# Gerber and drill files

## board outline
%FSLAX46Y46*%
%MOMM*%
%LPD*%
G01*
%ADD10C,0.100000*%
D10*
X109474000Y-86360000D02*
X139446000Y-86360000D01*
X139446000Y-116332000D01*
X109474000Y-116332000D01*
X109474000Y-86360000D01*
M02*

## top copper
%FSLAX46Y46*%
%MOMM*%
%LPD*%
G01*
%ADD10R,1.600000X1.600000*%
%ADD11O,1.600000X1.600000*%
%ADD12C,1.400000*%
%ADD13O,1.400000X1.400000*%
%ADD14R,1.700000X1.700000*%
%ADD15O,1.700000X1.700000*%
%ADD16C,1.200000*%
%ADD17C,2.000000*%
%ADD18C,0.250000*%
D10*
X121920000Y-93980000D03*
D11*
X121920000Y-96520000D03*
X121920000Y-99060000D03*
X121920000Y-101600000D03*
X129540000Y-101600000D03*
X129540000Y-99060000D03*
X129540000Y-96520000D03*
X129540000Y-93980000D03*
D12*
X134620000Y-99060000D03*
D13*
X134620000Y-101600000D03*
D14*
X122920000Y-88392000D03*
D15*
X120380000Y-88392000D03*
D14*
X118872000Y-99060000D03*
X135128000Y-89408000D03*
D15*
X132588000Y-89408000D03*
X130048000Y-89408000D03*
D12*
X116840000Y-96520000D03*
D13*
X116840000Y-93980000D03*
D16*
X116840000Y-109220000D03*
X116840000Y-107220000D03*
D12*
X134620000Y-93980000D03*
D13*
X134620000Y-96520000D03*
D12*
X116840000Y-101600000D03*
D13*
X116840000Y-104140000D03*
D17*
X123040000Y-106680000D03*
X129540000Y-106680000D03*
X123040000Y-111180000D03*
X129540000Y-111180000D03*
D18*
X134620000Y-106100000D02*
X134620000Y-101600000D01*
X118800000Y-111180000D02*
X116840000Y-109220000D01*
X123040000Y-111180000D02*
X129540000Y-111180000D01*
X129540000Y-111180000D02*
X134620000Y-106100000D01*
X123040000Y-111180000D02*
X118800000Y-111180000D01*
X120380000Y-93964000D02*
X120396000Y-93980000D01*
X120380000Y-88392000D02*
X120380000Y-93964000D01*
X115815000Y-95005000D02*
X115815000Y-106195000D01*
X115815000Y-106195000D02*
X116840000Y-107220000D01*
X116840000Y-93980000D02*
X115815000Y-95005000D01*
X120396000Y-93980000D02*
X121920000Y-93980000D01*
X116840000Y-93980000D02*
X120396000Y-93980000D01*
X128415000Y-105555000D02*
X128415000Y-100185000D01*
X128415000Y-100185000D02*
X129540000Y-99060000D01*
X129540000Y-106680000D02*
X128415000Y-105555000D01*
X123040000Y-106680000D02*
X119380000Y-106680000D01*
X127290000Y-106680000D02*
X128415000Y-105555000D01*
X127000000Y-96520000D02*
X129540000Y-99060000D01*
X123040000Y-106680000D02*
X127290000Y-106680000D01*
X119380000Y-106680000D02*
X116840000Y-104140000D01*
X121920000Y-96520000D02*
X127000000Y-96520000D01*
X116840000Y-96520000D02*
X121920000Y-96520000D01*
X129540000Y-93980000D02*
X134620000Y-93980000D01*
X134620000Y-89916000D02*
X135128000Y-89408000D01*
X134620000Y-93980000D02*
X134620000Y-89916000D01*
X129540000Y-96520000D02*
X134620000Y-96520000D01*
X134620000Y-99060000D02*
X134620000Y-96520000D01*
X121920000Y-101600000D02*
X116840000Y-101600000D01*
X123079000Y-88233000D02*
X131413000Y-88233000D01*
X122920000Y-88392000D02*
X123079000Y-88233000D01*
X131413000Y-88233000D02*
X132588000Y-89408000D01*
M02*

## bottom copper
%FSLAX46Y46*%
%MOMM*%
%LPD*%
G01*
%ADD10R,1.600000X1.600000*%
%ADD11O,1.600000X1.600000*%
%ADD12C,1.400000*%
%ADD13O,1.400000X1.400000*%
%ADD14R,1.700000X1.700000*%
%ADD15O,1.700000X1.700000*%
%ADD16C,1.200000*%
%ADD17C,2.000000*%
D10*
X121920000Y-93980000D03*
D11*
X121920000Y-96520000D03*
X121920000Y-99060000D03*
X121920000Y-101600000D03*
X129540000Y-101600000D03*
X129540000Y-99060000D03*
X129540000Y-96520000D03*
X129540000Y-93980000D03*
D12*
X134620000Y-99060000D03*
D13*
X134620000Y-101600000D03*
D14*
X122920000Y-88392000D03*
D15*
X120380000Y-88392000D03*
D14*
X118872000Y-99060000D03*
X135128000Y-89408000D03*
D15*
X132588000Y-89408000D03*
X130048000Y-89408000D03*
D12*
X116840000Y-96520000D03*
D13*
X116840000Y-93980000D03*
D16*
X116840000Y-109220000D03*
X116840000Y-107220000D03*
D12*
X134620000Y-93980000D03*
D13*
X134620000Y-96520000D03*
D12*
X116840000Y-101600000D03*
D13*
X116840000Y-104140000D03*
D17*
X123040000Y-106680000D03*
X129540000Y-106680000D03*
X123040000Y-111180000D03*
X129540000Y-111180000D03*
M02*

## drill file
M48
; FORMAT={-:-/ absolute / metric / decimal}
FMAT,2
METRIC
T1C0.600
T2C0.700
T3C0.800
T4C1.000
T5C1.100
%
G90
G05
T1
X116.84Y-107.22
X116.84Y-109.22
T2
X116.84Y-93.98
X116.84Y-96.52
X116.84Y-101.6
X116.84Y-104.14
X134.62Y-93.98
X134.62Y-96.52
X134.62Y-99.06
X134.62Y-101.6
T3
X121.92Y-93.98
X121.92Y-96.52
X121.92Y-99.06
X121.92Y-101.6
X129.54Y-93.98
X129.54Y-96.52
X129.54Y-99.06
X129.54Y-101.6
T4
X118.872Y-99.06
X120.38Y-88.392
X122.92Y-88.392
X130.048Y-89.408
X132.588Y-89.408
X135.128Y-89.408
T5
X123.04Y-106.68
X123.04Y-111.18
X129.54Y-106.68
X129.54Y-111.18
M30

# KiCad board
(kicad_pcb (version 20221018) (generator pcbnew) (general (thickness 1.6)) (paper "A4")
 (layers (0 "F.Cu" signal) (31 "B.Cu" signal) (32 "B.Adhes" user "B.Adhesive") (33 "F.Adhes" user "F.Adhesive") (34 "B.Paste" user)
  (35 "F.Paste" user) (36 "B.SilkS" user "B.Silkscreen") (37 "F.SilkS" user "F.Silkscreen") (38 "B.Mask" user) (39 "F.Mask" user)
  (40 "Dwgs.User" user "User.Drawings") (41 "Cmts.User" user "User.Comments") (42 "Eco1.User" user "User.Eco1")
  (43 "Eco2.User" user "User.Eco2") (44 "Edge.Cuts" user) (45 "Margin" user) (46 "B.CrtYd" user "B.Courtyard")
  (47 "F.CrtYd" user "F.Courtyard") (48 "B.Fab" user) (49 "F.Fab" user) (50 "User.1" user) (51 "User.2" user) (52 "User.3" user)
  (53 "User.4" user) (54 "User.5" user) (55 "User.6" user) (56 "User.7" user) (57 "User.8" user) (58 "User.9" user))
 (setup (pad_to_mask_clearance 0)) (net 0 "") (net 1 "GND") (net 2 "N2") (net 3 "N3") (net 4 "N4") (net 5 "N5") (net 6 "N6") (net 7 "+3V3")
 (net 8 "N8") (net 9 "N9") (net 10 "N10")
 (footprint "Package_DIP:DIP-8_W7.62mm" (layer "F.Cu") (at 121.92 93.98)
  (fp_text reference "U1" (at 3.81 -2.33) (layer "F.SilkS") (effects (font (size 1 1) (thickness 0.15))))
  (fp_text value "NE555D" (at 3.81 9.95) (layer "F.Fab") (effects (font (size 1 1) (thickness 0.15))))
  (pad "1" thru_hole rect (at 0 0) (size 1.6 1.6) (drill 0.8) (layers "*.Cu" "*.Mask") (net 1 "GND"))
  (pad "2" thru_hole oval (at 0 2.54) (size 1.6 1.6) (drill 0.8) (layers "*.Cu" "*.Mask") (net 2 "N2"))
  (pad "3" thru_hole oval (at 0 5.08) (size 1.6 1.6) (drill 0.8) (layers "*.Cu" "*.Mask") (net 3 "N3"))
  (pad "4" thru_hole oval (at 0 7.62) (size 1.6 1.6) (drill 0.8) (layers "*.Cu" "*.Mask") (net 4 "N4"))
  (pad "5" thru_hole oval (at 7.62 7.62) (size 1.6 1.6) (drill 0.8) (layers "*.Cu" "*.Mask") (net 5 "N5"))
  (pad "6" thru_hole oval (at 7.62 5.08) (size 1.6 1.6) (drill 0.8) (layers "*.Cu" "*.Mask") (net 2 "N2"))
  (pad "7" thru_hole oval (at 7.62 2.54) (size 1.6 1.6) (drill 0.8) (layers "*.Cu" "*.Mask") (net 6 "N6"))
  (pad "8" thru_hole oval (at 7.62 0) (size 1.6 1.6) (drill 0.8) (layers "*.Cu" "*.Mask") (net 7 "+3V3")))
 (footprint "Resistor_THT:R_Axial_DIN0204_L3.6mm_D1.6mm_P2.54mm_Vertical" (layer "F.Cu") (at 134.62 99.06 -90)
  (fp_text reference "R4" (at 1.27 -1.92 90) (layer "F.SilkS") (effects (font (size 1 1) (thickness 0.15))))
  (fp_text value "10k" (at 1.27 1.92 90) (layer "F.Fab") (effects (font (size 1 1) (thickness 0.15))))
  (pad "1" thru_hole circle (at 0 0 270) (size 1.4 1.4) (drill 0.7) (layers "*.Cu" "*.Mask") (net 6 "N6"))
  (pad "2" thru_hole oval (at 2.54 0 270) (size 1.4 1.4) (drill 0.7) (layers "*.Cu" "*.Mask") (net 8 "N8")))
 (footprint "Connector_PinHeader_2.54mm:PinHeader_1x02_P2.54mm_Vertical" (layer "F.Cu") (at 122.92 88.392 -90)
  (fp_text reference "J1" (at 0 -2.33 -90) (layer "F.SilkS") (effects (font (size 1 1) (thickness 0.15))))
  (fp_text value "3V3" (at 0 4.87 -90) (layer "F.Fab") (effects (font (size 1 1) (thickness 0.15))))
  (pad "1" thru_hole rect (at 0 0 270) (size 1.7 1.7) (drill 1) (layers "*.Cu" "*.Mask") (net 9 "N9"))
  (pad "2" thru_hole oval (at 0 2.54 270) (size 1.7 1.7) (drill 1) (layers "*.Cu" "*.Mask") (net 1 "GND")))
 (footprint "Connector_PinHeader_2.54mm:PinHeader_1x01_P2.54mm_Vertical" (layer "F.Cu") (at 118.872 99.06)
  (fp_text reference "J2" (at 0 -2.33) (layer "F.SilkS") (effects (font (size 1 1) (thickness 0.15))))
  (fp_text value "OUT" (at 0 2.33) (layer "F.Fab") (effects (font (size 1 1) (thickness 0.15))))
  (pad "1" thru_hole rect (at 0 0) (size 1.7 1.7) (drill 1) (layers "*.Cu" "*.Mask") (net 3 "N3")))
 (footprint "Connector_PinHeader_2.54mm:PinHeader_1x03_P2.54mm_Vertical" (layer "F.Cu") (at 135.128 89.408 -90)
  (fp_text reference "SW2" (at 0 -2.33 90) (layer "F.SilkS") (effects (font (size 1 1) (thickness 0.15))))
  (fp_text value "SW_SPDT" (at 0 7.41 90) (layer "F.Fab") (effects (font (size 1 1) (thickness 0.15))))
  (pad "1" thru_hole rect (at 0 0 270) (size 1.7 1.7) (drill 1) (layers "*.Cu" "*.Mask") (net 7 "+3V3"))
  (pad "2" thru_hole oval (at 0 2.54 270) (size 1.7 1.7) (drill 1) (layers "*.Cu" "*.Mask") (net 9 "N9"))
  (pad "3" thru_hole oval (at 0 5.08 270) (size 1.7 1.7) (drill 1) (layers "*.Cu" "*.Mask") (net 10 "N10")))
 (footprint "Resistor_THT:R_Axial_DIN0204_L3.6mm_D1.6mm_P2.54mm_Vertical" (layer "F.Cu") (at 116.84 96.52 90)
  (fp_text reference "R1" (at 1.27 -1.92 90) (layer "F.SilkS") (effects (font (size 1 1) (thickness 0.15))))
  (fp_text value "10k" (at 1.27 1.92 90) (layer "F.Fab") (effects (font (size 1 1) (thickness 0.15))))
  (pad "1" thru_hole circle (at 0 0 90) (size 1.4 1.4) (drill 0.7) (layers "*.Cu" "*.Mask") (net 2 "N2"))
  (pad "2" thru_hole oval (at 2.54 0 90) (size 1.4 1.4) (drill 0.7) (layers "*.Cu" "*.Mask") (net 1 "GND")))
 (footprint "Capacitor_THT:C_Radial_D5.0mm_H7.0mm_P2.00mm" (layer "F.Cu") (at 116.84 109.22 90)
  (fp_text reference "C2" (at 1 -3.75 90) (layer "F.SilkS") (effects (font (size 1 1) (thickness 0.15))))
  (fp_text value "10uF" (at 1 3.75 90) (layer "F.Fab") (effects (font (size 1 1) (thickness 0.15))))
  (pad "1" thru_hole circle (at 0 0 90) (size 1.2 1.2) (drill 0.6) (layers "*.Cu" "*.Mask") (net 8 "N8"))
  (pad "2" thru_hole circle (at 2 0 90) (size 1.2 1.2) (drill 0.6) (layers "*.Cu" "*.Mask") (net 1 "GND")))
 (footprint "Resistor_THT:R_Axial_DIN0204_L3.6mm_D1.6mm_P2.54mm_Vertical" (layer "F.Cu") (at 134.62 93.98 -90)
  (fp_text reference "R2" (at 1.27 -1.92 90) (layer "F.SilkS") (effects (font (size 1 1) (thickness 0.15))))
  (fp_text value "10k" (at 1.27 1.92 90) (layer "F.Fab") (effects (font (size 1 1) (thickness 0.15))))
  (pad "1" thru_hole circle (at 0 0 270) (size 1.4 1.4) (drill 0.7) (layers "*.Cu" "*.Mask") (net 7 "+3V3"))
  (pad "2" thru_hole oval (at 2.54 0 270) (size 1.4 1.4) (drill 0.7) (layers "*.Cu" "*.Mask") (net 6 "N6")))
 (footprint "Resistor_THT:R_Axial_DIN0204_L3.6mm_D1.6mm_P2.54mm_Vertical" (layer "F.Cu") (at 116.84 101.6 -90)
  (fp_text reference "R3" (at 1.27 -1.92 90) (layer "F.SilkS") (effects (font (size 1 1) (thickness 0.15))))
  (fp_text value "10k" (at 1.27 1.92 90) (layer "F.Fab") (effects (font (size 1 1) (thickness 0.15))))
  (pad "1" thru_hole circle (at 0 0 270) (size 1.4 1.4) (drill 0.7) (layers "*.Cu" "*.Mask") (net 4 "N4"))
  (pad "2" thru_hole oval (at 2.54 0 270) (size 1.4 1.4) (drill 0.7) (layers "*.Cu" "*.Mask") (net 2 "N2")))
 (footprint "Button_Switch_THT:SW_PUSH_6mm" (layer "F.Cu") (at 123.04 106.68)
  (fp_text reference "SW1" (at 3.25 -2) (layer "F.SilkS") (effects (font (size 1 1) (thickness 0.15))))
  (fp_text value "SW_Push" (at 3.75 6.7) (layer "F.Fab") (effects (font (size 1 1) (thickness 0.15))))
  (pad "1" thru_hole circle (at 0 0 90) (size 2 2) (drill 1.1) (layers "*.Cu" "*.Mask") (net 2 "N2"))
  (pad "1" thru_hole circle (at 6.5 0 90) (size 2 2) (drill 1.1) (layers "*.Cu" "*.Mask") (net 2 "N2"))
  (pad "2" thru_hole circle (at 0 4.5 90) (size 2 2) (drill 1.1) (layers "*.Cu" "*.Mask") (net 8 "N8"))
  (pad "2" thru_hole circle (at 6.5 4.5 90) (size 2 2) (drill 1.1) (layers "*.Cu" "*.Mask") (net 8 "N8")))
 (gr_rect (start 109.474 86.36) (end 139.446 116.332) (stroke (width 0.1) (type default)) (fill none) (layer "Edge.Cuts"))
 (segment (start 134.62 106.1) (end 134.62 101.6) (width 0.25) (layer "F.Cu") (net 8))
 (segment (start 118.8 111.18) (end 116.84 109.22) (width 0.25) (layer "F.Cu") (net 8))
 (segment (start 123.04 111.18) (end 129.54 111.18) (width 0.25) (layer "F.Cu") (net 8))
 (segment (start 129.54 111.18) (end 134.62 106.1) (width 0.25) (layer "F.Cu") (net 8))
 (segment (start 123.04 111.18) (end 118.8 111.18) (width 0.25) (layer "F.Cu") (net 8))
 (segment (start 120.38 93.964) (end 120.396 93.98) (width 0.25) (layer "F.Cu") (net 1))
 (segment (start 120.38 88.392) (end 120.38 93.964) (width 0.25) (layer "F.Cu") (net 1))
 (segment (start 115.815 95.005) (end 115.815 106.195) (width 0.25) (layer "F.Cu") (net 1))
 (segment (start 115.815 106.195) (end 116.84 107.22) (width 0.25) (layer "F.Cu") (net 1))
 (segment (start 116.84 93.98) (end 115.815 95.005) (width 0.25) (layer "F.Cu") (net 1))
 (segment (start 120.396 93.98) (end 121.92 93.98) (width 0.25) (layer "F.Cu") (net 1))
 (segment (start 116.84 93.98) (end 120.396 93.98) (width 0.25) (layer "F.Cu") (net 1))
 (segment (start 128.415 105.555) (end 128.415 100.185) (width 0.25) (layer "F.Cu") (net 2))
 (segment (start 128.415 100.185) (end 129.54 99.06) (width 0.25) (layer "F.Cu") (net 2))
 (segment (start 129.54 106.68) (end 128.415 105.555) (width 0.25) (layer "F.Cu") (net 2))
 (segment (start 123.04 106.68) (end 119.38 106.68) (width 0.25) (layer "F.Cu") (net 2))
 (segment (start 127.29 106.68) (end 128.415 105.555) (width 0.25) (layer "F.Cu") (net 2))
 (segment (start 127 96.52) (end 129.54 99.06) (width 0.25) (layer "F.Cu") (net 2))
 (segment (start 123.04 106.68) (end 127.29 106.68) (width 0.25) (layer "F.Cu") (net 2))
 (segment (start 119.38 106.68) (end 116.84 104.14) (width 0.25) (layer "F.Cu") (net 2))
 (segment (start 121.92 96.52) (end 127 96.52) (width 0.25) (layer "F.Cu") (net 2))
 (segment (start 116.84 96.52) (end 121.92 96.52) (width 0.25) (layer "F.Cu") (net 2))
 (segment (start 129.54 93.98) (end 134.62 93.98) (width 0.25) (layer "F.Cu") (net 7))
 (segment (start 134.62 89.916) (end 135.128 89.408) (width 0.25) (layer "F.Cu") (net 7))
 (segment (start 134.62 93.98) (end 134.62 89.916) (width 0.25) (layer "F.Cu") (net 7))
 (segment (start 129.54 96.52) (end 134.62 96.52) (width 0.25) (layer "F.Cu") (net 6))
 (segment (start 134.62 99.06) (end 134.62 96.52) (width 0.25) (layer "F.Cu") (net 6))
 (segment (start 121.92 101.6) (end 116.84 101.6) (width 0.25) (layer "F.Cu") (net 4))
 (segment (start 123.079 88.233) (end 131.413 88.233) (width 0.25) (layer "F.Cu") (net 9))
 (segment (start 122.92 88.392) (end 123.079 88.233) (width 0.25) (layer "F.Cu") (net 9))
 (segment (start 131.413 88.233) (end 132.588 89.408) (width 0.25) (layer "F.Cu") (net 9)))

